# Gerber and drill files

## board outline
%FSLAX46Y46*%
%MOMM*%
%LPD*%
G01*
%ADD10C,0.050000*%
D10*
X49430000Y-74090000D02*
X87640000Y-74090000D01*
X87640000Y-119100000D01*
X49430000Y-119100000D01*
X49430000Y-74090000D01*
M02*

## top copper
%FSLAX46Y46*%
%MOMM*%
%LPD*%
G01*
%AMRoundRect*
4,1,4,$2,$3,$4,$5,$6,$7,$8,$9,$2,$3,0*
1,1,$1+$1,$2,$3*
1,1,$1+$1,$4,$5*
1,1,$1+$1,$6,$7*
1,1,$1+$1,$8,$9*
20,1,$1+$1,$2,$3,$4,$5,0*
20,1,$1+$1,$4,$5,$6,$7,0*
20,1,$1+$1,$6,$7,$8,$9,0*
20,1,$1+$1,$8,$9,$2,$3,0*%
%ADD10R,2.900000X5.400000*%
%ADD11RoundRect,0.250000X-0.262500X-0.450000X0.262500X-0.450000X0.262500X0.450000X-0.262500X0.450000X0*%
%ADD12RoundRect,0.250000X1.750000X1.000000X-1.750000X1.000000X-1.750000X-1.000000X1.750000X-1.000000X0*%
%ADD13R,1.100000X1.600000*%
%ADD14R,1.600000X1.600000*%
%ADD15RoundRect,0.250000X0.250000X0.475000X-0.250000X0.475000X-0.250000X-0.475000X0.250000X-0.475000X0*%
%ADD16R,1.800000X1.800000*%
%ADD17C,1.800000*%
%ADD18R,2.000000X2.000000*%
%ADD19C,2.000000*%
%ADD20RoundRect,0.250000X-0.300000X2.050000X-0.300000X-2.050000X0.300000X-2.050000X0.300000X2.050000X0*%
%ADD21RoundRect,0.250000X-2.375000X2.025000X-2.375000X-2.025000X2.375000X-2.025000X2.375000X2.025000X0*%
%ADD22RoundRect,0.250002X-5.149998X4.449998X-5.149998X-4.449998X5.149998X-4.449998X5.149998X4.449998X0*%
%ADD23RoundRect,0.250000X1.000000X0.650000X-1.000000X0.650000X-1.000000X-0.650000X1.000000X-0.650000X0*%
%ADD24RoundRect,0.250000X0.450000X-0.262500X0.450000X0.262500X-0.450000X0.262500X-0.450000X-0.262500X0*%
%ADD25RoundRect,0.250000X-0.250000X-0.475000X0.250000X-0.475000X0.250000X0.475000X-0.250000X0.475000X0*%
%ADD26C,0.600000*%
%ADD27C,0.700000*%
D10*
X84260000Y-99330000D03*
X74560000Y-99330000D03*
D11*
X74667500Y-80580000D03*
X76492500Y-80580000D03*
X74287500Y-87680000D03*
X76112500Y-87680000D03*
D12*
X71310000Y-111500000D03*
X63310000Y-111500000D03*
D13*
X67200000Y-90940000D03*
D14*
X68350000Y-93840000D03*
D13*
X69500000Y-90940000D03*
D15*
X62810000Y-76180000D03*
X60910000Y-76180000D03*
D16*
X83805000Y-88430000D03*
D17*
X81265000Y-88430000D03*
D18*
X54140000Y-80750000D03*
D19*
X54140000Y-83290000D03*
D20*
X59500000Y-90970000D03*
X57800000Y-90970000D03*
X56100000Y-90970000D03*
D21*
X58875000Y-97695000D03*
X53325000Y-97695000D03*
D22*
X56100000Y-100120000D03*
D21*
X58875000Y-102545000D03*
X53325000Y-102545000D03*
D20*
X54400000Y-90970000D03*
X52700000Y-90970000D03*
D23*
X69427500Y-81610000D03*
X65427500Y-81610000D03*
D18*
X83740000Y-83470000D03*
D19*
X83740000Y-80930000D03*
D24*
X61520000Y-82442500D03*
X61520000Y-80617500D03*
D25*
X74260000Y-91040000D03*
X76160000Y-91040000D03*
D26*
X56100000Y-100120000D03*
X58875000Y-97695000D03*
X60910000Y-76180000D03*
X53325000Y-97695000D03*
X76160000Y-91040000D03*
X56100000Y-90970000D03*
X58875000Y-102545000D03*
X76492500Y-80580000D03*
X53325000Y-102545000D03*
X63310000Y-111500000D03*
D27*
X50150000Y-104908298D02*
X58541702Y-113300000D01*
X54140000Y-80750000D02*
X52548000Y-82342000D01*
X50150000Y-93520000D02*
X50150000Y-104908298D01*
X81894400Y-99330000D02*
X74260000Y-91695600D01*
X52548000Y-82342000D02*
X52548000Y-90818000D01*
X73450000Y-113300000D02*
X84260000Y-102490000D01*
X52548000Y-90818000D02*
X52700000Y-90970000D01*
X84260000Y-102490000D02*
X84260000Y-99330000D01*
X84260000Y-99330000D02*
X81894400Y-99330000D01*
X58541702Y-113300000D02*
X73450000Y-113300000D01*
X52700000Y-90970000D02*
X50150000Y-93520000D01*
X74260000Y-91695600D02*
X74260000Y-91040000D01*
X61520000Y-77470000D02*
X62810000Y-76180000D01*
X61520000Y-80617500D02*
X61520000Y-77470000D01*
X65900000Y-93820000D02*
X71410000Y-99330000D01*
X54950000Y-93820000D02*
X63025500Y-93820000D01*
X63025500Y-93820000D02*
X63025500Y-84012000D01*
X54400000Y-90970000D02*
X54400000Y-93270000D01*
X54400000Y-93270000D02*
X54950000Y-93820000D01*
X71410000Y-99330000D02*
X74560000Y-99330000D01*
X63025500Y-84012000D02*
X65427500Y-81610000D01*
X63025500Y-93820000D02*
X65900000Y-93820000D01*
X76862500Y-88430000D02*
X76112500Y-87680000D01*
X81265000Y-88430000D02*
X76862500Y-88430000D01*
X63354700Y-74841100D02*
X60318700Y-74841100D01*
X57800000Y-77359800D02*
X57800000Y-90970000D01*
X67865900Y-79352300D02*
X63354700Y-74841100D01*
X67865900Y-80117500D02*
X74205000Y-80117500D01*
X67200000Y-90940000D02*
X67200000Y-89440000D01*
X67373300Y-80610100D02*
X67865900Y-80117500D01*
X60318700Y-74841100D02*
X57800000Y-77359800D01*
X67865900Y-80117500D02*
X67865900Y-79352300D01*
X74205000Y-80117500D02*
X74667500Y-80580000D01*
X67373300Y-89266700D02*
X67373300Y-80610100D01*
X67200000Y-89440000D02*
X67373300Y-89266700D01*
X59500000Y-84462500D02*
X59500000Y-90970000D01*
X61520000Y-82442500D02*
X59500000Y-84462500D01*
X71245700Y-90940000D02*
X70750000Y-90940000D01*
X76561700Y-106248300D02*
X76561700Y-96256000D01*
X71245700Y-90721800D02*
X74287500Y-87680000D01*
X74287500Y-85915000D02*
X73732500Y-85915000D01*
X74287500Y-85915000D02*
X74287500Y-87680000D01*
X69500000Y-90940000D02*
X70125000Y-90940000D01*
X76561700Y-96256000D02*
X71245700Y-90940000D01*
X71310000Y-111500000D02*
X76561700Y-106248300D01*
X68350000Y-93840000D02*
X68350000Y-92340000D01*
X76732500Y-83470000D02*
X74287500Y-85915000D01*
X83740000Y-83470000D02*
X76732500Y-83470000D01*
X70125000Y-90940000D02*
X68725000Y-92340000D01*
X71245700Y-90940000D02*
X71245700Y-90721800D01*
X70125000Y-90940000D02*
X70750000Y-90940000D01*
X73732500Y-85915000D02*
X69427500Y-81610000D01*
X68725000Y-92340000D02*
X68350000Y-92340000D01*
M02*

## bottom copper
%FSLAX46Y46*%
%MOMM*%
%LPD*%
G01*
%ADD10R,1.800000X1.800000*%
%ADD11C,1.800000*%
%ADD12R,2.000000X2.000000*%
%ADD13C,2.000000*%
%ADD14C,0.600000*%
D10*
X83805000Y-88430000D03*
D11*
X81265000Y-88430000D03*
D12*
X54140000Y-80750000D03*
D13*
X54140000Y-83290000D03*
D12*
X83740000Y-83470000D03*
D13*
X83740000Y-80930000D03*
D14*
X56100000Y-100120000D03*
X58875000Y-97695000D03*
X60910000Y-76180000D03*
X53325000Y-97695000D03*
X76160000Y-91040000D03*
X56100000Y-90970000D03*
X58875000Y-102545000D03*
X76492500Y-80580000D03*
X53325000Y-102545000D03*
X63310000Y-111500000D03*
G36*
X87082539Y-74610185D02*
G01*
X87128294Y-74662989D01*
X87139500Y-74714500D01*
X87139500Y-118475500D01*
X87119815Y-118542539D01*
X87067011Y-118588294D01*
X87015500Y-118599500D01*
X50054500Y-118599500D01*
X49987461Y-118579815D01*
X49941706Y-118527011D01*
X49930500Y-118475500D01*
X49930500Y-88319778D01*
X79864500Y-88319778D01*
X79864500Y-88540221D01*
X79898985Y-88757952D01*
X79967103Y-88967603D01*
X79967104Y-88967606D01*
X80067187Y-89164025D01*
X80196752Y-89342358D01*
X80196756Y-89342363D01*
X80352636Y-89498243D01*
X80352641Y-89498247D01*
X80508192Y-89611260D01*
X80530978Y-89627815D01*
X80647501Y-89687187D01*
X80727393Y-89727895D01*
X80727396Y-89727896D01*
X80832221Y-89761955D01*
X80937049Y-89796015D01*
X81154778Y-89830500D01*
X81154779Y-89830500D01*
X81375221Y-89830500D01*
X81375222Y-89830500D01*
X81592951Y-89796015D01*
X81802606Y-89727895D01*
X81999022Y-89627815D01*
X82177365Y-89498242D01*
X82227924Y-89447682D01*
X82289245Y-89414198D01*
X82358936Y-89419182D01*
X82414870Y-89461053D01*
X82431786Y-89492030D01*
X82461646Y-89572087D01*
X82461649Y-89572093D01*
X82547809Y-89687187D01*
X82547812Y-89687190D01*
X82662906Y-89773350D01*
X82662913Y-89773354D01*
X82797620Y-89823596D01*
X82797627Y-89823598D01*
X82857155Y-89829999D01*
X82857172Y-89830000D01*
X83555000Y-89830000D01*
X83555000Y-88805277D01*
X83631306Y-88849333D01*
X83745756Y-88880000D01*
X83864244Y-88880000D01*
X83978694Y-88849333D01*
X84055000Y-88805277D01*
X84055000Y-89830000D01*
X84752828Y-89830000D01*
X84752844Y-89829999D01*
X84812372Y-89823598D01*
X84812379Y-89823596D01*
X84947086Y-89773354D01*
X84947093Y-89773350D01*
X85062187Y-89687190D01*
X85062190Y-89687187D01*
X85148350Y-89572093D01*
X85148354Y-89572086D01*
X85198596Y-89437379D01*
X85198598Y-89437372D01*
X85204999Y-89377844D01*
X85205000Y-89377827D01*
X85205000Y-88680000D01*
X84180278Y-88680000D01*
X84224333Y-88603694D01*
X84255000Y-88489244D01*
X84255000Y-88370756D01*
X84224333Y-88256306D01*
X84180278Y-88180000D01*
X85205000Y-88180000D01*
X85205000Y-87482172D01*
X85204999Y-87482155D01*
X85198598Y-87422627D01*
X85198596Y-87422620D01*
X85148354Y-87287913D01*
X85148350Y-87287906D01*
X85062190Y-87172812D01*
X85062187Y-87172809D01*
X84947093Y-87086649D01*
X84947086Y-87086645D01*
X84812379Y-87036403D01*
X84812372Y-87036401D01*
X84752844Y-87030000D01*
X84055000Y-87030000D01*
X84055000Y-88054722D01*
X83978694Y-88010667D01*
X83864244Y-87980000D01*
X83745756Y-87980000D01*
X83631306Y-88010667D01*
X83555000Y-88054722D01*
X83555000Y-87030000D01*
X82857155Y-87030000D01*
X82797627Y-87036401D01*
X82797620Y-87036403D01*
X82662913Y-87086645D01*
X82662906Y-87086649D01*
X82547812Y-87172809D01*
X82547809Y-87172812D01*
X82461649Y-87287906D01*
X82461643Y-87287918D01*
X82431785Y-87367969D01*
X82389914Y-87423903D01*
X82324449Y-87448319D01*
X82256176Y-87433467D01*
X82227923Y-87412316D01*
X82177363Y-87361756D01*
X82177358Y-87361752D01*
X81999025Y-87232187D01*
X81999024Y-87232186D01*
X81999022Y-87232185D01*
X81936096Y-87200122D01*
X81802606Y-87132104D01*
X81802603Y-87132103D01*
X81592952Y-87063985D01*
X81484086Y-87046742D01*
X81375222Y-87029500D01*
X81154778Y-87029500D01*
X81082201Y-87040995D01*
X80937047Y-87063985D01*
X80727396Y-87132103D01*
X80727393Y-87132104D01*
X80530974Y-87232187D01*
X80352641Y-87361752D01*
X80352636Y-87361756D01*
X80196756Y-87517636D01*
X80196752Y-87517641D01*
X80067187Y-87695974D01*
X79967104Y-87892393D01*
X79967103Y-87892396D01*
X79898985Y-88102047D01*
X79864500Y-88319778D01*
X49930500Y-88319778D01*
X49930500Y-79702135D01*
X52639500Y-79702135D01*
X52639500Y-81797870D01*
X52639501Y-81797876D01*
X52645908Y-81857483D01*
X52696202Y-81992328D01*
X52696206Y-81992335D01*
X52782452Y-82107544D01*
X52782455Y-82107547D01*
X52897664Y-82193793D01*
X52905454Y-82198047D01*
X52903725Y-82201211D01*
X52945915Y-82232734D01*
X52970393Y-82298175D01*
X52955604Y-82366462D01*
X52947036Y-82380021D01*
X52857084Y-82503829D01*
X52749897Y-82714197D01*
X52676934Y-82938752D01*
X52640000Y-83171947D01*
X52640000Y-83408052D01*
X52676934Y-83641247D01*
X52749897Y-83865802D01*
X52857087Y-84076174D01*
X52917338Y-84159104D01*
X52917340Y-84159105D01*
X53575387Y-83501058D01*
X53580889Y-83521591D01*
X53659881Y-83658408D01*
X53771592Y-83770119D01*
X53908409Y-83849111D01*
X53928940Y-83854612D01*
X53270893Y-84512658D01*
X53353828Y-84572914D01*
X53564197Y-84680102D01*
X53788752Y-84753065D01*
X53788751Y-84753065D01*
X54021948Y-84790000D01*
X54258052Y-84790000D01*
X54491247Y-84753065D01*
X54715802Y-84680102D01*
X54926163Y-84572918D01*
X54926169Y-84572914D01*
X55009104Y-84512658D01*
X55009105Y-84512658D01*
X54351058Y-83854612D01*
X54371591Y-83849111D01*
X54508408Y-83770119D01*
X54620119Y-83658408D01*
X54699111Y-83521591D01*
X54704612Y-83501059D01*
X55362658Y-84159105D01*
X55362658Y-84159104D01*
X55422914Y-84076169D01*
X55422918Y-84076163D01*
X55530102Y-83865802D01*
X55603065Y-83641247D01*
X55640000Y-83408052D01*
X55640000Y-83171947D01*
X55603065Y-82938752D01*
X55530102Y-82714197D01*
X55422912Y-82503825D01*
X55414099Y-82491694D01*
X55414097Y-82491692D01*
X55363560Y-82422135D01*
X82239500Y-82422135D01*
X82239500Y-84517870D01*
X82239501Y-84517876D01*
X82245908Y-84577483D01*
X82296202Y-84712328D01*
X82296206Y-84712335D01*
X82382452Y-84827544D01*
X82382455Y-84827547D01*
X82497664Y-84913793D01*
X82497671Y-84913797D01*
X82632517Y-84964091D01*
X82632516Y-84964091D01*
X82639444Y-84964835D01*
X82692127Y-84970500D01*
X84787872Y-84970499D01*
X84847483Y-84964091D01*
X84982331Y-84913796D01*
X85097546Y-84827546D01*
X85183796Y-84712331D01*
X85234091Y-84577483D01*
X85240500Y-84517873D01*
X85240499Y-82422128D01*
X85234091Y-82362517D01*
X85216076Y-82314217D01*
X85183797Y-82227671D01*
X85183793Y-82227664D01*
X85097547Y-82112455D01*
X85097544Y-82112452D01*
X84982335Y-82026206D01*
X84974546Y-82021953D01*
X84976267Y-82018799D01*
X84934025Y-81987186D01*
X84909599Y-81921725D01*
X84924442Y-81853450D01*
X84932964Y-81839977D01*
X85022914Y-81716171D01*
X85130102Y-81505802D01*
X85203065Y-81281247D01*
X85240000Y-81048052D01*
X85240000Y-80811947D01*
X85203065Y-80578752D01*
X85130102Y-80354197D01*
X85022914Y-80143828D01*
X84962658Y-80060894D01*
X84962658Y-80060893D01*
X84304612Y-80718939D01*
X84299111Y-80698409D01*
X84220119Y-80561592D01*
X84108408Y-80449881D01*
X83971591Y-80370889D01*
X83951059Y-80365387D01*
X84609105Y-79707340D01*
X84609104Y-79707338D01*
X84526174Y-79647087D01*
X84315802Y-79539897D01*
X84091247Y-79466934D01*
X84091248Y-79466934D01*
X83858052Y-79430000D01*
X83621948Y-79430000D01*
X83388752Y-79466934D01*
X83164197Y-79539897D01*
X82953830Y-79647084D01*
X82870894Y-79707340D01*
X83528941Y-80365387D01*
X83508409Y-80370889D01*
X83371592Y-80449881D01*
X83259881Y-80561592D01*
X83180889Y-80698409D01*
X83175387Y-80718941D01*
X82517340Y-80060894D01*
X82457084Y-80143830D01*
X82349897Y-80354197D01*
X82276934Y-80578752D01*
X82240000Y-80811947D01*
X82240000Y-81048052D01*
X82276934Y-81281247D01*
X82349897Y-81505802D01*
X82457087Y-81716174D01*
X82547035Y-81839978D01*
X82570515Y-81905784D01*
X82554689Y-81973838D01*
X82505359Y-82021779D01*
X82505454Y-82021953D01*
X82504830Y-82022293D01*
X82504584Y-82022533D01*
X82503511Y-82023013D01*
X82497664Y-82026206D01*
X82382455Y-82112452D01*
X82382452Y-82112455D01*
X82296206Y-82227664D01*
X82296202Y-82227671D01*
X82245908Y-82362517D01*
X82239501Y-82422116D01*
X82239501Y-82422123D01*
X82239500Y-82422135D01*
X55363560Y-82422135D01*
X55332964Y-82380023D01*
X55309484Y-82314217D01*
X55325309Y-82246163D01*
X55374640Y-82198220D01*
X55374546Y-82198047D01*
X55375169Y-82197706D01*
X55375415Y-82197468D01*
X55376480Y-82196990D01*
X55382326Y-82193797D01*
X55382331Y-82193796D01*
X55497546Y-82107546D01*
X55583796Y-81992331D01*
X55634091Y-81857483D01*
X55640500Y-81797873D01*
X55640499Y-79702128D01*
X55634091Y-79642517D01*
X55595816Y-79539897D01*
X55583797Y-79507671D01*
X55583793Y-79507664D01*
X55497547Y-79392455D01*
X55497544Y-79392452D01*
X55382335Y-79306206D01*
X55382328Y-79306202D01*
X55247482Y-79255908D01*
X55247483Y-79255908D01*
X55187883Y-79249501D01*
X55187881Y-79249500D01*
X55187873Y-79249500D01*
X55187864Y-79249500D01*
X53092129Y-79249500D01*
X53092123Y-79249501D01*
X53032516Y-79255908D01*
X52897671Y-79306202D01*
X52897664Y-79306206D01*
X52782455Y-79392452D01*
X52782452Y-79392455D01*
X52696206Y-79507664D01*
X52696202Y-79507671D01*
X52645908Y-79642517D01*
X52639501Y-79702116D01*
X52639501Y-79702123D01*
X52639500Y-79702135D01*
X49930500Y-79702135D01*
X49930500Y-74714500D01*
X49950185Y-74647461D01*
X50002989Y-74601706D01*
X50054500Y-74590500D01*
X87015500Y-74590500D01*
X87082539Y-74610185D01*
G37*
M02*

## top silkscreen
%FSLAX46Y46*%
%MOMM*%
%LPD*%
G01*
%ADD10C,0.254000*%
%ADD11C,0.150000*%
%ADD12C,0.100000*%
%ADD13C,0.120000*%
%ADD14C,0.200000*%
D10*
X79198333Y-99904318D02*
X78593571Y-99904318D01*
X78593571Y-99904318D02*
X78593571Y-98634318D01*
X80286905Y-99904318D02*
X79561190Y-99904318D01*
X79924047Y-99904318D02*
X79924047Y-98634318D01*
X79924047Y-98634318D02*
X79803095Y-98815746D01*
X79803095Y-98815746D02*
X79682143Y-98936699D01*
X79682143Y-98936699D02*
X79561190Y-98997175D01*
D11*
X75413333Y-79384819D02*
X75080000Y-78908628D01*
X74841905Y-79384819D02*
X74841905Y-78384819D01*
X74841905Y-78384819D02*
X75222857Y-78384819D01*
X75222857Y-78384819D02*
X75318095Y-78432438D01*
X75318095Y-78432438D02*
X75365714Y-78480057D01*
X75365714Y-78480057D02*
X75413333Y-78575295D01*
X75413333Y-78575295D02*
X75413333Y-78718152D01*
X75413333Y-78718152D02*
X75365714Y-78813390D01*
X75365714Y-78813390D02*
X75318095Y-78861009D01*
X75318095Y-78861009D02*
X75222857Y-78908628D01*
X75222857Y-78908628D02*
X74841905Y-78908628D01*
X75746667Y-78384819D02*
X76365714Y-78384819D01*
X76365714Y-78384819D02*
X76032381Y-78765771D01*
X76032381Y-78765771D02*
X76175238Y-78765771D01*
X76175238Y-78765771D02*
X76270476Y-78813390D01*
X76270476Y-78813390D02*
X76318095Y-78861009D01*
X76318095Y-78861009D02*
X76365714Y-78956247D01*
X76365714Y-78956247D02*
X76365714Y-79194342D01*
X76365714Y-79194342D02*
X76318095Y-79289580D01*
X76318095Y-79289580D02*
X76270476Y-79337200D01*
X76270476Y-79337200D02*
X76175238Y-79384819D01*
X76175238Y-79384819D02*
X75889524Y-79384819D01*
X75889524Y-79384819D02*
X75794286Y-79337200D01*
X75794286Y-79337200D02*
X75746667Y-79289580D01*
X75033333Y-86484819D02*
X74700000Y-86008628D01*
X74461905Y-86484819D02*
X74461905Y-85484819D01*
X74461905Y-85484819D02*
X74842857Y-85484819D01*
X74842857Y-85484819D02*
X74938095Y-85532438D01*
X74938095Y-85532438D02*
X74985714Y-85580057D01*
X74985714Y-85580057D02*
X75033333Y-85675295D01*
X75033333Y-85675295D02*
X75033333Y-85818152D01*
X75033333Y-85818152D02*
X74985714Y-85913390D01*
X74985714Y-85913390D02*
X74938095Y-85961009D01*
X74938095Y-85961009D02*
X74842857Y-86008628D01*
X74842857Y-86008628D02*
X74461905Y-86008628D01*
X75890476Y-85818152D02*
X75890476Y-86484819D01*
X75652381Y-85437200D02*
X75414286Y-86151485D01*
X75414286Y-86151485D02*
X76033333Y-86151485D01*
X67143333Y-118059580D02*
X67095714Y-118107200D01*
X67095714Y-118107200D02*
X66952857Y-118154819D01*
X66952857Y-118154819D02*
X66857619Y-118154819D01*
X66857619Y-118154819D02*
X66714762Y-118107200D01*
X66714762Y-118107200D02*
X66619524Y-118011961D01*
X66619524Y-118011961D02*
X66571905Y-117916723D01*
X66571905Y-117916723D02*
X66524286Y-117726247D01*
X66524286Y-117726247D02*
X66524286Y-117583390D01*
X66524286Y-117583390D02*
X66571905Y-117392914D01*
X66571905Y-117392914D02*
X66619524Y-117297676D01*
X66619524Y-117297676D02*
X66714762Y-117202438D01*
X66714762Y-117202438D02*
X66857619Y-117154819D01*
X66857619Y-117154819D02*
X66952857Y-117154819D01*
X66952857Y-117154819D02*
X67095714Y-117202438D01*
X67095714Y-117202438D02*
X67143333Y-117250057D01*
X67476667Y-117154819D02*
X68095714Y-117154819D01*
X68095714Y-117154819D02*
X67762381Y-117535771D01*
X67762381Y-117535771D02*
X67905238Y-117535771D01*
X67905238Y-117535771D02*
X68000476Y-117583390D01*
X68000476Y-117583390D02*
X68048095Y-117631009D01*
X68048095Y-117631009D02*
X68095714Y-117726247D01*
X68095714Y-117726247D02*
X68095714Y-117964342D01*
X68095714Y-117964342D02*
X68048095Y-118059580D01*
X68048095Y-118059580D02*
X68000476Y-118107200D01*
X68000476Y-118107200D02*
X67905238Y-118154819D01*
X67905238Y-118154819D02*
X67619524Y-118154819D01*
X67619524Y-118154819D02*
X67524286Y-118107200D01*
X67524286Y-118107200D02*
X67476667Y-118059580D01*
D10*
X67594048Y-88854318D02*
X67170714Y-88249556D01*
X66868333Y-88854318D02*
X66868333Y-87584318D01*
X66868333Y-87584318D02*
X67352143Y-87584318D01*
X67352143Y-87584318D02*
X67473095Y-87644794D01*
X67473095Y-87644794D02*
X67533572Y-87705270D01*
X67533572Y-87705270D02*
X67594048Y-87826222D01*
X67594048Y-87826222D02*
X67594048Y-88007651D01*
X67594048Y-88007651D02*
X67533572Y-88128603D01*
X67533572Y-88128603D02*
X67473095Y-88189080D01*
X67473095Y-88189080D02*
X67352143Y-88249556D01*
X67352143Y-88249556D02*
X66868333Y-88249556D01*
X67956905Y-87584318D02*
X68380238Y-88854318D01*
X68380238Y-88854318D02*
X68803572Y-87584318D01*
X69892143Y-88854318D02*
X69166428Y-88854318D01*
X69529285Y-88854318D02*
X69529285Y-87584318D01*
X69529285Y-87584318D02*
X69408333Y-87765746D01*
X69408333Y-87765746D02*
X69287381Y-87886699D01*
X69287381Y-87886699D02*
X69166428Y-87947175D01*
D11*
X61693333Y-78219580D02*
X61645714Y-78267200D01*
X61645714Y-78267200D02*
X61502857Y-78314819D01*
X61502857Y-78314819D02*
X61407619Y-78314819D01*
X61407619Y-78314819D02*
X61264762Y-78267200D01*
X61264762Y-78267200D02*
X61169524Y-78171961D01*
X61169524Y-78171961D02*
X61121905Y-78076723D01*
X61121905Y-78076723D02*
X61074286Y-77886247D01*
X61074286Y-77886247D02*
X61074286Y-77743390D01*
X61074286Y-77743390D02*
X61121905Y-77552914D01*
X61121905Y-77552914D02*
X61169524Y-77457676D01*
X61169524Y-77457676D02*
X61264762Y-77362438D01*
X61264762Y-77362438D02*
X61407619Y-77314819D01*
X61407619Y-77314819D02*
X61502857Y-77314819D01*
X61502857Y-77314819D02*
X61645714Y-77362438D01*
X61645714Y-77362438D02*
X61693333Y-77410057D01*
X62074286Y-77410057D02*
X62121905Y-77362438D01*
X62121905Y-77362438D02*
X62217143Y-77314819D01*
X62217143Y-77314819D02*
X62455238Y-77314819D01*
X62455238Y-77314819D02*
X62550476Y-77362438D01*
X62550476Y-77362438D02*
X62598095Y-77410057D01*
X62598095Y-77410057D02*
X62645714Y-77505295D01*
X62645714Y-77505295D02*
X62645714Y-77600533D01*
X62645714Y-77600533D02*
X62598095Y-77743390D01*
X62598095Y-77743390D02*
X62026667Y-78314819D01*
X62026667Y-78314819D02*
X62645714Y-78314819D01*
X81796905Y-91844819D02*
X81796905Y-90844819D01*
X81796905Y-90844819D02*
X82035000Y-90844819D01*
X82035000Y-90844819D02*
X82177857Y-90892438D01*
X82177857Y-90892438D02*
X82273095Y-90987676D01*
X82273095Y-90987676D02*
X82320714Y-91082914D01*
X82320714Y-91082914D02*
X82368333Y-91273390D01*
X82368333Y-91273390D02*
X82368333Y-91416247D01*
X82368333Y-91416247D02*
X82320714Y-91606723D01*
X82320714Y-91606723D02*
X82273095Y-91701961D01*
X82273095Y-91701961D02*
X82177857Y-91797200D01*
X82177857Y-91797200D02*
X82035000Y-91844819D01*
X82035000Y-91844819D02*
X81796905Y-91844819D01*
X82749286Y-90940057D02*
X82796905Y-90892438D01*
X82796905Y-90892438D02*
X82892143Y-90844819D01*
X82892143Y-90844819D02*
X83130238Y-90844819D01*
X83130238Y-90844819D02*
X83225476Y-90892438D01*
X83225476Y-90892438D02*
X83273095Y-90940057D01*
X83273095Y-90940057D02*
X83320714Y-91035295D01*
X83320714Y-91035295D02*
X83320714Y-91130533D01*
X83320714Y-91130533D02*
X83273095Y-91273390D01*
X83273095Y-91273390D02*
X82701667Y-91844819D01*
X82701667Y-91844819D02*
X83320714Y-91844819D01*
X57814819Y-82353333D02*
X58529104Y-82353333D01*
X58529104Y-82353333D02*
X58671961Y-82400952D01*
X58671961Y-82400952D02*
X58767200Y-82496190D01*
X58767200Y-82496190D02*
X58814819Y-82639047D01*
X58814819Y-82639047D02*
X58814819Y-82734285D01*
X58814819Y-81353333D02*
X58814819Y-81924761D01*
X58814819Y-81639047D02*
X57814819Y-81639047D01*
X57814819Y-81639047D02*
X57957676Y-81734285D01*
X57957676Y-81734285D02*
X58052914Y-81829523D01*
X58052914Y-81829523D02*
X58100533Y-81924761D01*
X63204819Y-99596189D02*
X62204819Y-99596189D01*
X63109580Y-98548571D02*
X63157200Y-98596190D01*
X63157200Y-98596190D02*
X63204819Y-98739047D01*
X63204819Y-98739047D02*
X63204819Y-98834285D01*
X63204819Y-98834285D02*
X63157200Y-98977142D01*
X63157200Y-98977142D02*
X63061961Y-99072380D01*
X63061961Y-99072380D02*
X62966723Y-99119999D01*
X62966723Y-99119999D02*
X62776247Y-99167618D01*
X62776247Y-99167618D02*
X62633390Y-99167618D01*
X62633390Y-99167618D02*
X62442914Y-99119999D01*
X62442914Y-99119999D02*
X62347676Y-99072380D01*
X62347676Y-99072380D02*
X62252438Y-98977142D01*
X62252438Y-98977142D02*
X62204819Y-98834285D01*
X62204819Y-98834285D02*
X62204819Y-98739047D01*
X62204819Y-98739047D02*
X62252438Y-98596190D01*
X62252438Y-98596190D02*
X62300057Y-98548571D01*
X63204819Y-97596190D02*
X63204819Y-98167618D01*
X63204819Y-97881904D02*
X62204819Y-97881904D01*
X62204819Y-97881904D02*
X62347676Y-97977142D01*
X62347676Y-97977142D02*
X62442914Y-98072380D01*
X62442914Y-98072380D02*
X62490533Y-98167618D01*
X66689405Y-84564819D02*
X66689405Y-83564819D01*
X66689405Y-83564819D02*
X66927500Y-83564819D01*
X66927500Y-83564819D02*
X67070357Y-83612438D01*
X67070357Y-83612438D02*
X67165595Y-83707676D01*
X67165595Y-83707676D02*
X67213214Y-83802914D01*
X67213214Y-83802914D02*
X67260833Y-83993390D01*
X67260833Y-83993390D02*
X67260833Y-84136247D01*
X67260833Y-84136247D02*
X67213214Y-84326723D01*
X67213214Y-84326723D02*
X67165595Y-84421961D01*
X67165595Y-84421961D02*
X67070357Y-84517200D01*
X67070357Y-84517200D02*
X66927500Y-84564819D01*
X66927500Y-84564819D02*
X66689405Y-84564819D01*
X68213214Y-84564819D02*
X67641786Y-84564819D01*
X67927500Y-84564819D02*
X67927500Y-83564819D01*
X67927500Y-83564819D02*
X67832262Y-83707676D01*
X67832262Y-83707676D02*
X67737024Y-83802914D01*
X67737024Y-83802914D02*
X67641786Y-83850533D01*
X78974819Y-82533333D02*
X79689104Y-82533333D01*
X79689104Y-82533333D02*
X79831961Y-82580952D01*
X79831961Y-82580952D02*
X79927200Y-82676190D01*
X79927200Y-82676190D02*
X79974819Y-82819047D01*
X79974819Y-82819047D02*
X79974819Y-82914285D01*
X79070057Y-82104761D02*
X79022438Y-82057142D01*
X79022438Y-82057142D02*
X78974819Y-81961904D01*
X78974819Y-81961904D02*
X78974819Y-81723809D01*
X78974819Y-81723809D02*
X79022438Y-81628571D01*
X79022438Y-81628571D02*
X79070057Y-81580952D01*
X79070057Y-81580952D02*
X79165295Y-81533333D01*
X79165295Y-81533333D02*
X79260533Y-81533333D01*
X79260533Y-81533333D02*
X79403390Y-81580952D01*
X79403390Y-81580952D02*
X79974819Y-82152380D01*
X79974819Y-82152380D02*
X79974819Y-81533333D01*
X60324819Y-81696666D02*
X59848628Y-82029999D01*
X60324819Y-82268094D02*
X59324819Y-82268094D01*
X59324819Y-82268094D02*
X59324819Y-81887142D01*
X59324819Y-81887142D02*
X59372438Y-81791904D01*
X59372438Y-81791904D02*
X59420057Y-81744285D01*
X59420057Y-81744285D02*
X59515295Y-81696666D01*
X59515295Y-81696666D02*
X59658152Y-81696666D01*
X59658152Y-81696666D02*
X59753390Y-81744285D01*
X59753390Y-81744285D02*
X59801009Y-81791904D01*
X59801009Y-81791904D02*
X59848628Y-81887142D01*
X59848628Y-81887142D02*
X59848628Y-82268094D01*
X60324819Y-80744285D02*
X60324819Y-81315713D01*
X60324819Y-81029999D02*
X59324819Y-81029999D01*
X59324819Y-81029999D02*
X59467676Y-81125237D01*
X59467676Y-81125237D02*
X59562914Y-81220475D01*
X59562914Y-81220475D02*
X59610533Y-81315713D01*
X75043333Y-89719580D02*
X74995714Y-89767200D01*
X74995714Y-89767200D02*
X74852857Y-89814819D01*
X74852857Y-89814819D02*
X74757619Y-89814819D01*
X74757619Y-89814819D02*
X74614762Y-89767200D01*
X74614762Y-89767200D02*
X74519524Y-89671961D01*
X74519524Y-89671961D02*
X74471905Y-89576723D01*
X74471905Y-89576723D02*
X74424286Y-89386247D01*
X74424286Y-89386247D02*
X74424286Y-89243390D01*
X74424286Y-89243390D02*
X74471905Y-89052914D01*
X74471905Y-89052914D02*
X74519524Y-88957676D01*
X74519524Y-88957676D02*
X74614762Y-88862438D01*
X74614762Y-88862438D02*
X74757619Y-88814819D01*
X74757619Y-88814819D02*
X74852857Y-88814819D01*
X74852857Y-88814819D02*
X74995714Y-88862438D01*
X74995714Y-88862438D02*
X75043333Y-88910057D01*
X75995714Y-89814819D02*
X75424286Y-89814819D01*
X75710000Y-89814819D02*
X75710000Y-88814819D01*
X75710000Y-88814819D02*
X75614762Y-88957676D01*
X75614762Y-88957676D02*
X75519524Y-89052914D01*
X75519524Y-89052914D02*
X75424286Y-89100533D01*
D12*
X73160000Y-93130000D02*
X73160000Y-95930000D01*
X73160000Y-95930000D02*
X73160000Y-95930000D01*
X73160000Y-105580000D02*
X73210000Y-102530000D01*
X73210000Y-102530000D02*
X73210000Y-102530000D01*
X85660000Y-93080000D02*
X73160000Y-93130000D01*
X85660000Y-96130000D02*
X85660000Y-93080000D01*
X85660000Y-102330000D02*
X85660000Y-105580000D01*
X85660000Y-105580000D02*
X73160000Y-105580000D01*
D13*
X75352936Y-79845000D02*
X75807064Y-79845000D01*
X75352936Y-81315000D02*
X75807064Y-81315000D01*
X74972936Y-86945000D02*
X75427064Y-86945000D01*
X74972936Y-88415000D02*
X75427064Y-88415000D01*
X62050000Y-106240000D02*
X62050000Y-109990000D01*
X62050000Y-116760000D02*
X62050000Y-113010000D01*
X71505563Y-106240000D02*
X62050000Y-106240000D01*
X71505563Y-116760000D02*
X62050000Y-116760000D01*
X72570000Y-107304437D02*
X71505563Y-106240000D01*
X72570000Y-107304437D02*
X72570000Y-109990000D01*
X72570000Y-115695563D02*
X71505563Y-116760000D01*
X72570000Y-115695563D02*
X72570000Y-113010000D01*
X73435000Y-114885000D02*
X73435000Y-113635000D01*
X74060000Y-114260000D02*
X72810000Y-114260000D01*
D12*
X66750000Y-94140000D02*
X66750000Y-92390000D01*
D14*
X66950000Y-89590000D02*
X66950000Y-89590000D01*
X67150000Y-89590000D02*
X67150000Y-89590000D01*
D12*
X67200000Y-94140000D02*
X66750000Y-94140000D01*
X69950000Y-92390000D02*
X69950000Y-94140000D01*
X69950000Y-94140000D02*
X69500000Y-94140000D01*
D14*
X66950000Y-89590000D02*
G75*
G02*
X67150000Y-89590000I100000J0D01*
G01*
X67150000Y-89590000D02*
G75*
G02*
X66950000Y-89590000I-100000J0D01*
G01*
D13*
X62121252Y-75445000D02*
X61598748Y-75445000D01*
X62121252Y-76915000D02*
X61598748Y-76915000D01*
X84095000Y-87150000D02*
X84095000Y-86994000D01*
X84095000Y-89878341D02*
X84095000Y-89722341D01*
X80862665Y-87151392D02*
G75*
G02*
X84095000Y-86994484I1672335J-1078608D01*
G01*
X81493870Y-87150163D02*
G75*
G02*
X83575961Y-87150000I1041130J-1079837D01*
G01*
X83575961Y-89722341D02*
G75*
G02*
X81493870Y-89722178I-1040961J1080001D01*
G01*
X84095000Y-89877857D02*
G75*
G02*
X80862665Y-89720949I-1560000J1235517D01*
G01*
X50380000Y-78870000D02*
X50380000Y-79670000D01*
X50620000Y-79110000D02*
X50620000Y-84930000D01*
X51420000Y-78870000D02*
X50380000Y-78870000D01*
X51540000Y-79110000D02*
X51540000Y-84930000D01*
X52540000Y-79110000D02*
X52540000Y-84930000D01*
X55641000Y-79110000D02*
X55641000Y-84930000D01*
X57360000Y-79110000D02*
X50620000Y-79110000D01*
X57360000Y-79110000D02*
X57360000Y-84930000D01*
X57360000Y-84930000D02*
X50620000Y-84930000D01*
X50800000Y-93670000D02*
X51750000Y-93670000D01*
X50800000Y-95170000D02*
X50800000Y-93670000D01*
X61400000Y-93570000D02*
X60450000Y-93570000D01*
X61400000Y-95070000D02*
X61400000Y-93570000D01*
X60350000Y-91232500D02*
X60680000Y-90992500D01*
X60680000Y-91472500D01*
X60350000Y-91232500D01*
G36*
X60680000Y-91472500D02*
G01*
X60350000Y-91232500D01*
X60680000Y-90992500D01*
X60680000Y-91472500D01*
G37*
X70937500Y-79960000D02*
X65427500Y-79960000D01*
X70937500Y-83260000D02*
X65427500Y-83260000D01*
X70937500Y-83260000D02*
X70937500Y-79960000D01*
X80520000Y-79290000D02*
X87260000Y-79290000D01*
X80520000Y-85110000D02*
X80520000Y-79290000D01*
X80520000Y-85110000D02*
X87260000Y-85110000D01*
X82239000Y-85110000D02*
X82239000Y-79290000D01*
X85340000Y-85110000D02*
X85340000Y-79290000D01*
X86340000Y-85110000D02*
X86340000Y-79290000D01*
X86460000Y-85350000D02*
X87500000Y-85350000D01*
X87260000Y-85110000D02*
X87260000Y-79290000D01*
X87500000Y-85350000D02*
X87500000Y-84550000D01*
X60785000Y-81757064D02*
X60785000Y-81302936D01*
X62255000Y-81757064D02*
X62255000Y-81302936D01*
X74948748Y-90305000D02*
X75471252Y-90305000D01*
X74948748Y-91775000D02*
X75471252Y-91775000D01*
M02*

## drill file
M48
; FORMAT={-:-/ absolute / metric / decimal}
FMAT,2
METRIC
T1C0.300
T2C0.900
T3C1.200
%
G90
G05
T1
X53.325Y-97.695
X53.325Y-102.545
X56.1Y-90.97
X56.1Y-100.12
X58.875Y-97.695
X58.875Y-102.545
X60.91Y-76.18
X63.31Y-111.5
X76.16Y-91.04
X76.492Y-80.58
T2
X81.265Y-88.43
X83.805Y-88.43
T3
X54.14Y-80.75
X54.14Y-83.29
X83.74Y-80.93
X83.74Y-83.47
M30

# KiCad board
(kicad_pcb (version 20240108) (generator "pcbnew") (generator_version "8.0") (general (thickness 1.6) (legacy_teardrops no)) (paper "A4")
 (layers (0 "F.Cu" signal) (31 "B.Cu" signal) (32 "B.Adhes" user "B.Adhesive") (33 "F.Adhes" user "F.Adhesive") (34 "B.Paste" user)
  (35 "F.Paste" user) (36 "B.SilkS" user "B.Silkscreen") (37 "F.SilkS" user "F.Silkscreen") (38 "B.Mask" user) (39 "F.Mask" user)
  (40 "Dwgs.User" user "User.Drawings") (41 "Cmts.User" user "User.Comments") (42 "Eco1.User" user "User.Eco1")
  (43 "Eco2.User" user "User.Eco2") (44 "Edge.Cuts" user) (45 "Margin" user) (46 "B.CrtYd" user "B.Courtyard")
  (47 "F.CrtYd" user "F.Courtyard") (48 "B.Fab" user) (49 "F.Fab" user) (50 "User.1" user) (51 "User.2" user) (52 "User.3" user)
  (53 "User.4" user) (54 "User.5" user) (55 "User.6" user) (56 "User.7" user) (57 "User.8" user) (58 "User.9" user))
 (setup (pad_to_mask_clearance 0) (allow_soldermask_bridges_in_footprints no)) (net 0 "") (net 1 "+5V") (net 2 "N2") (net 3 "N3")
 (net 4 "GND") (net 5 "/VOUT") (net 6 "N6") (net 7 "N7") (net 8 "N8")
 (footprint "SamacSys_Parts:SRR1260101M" (layer "F.Cu") (at 79.41 99.33 180)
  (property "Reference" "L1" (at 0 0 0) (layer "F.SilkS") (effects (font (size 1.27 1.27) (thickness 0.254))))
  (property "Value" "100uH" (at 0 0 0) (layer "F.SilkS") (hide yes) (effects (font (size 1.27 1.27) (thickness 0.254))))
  (fp_line (start 6.25 6.2) (end 6.25 3.4) (stroke (width 0.1) (type solid)) (layer "F.SilkS"))
  (fp_line (start 6.25 3.4) (end 6.25 3.4) (stroke (width 0.1) (type solid)) (layer "F.SilkS"))
  (fp_line (start 6.25 -6.25) (end 6.2 -3.2) (stroke (width 0.1) (type solid)) (layer "F.SilkS"))
  (fp_line (start 6.2 -3.2) (end 6.2 -3.2) (stroke (width 0.1) (type solid)) (layer "F.SilkS"))
  (fp_line (start -6.25 6.25) (end 6.25 6.2) (stroke (width 0.1) (type solid)) (layer "F.SilkS"))
  (fp_line (start -6.25 3.2) (end -6.25 6.25) (stroke (width 0.1) (type solid)) (layer "F.SilkS"))
  (fp_line (start -6.25 -3) (end -6.25 -6.25) (stroke (width 0.1) (type solid)) (layer "F.SilkS"))
  (fp_line (start -6.25 -6.25) (end 6.25 -6.25) (stroke (width 0.1) (type solid)) (layer "F.SilkS"))
  (pad "1" smd rect (at -4.85 0 180) (size 2.9 5.4) (layers "F.Cu" "F.Paste" "F.Mask") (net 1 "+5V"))
  (pad "2" smd rect (at 4.85 0 180) (size 2.9 5.4) (layers "F.Cu" "F.Paste" "F.Mask") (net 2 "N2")))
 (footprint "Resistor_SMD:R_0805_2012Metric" (layer "F.Cu") (at 75.58 80.58)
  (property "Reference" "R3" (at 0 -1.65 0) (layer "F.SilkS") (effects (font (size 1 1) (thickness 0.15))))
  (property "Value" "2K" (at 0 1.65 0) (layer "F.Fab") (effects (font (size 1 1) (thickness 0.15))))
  (fp_line (start -0.227064 -0.735) (end 0.227064 -0.735) (stroke (width 0.12) (type solid)) (layer "F.SilkS"))
  (fp_line (start -0.227064 0.735) (end 0.227064 0.735) (stroke (width 0.12) (type solid)) (layer "F.SilkS"))
  (pad "1" smd roundrect (at -0.9125 0) (size 1.025 1.4) (layers "F.Cu" "F.Paste" "F.Mask") (roundrect_rratio 0.243902) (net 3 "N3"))
  (pad "2" smd roundrect (at 0.9125 0) (size 1.025 1.4) (layers "F.Cu" "F.Paste" "F.Mask") (roundrect_rratio 0.243902) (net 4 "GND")))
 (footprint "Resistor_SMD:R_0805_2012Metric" (layer "F.Cu") (at 75.2 87.68)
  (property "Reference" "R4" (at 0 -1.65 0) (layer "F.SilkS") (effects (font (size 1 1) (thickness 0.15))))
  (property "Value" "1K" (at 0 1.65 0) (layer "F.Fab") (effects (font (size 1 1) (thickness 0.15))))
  (fp_line (start -0.227064 -0.735) (end 0.227064 -0.735) (stroke (width 0.12) (type solid)) (layer "F.SilkS"))
  (fp_line (start -0.227064 0.735) (end 0.227064 0.735) (stroke (width 0.12) (type solid)) (layer "F.SilkS"))
  (pad "1" smd roundrect (at -0.9125 0) (size 1.025 1.4) (layers "F.Cu" "F.Paste" "F.Mask") (roundrect_rratio 0.243902) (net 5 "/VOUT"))
  (pad "2" smd roundrect (at 0.9125 0) (size 1.025 1.4) (layers "F.Cu" "F.Paste" "F.Mask") (roundrect_rratio 0.243902) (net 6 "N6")))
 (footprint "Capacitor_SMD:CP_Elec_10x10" (layer "F.Cu") (at 67.31 111.5 180)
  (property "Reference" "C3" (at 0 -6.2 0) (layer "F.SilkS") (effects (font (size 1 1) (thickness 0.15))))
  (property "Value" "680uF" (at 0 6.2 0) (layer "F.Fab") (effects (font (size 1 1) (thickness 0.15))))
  (fp_line (start 5.26 5.26) (end 5.26 1.51) (stroke (width 0.12) (type solid)) (layer "F.SilkS"))
  (fp_line (start 5.26 -5.26) (end 5.26 -1.51) (stroke (width 0.12) (type solid)) (layer "F.SilkS"))
  (fp_line (start -4.195563 5.26) (end 5.26 5.26) (stroke (width 0.12) (type solid)) (layer "F.SilkS"))
  (fp_line (start -4.195563 -5.26) (end 5.26 -5.26) (stroke (width 0.12) (type solid)) (layer "F.SilkS"))
  (fp_line (start -5.26 4.195563) (end -4.195563 5.26) (stroke (width 0.12) (type solid)) (layer "F.SilkS"))
  (fp_line (start -5.26 4.195563) (end -5.26 1.51) (stroke (width 0.12) (type solid)) (layer "F.SilkS"))
  (fp_line (start -5.26 -4.195563) (end -4.195563 -5.26) (stroke (width 0.12) (type solid)) (layer "F.SilkS"))
  (fp_line (start -5.26 -4.195563) (end -5.26 -1.51) (stroke (width 0.12) (type solid)) (layer "F.SilkS"))
  (fp_line (start -6.125 -3.385) (end -6.125 -2.135) (stroke (width 0.12) (type solid)) (layer "F.SilkS"))
  (fp_line (start -6.75 -2.76) (end -5.5 -2.76) (stroke (width 0.12) (type solid)) (layer "F.SilkS"))
  (pad "1" smd roundrect (at -4 0 180) (size 4 2.5) (layers "F.Cu" "F.Paste" "F.Mask") (roundrect_rratio 0.1) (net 5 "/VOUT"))
  (pad "2" smd roundrect (at 4 0 180) (size 4 2.5) (layers "F.Cu" "F.Paste" "F.Mask") (roundrect_rratio 0.1) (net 4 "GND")))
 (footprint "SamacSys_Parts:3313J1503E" (layer "F.Cu") (at 68.35 92.39 180)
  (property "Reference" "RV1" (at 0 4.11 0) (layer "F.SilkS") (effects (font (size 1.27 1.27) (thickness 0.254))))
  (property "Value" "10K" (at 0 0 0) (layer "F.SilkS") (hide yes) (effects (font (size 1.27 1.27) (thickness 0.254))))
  (fp_line (start 1.6 -1.75) (end 1.6 0) (stroke (width 0.1) (type solid)) (layer "F.SilkS"))
  (fp_line (start 1.4 2.8) (end 1.4 2.8) (stroke (width 0.2) (type solid)) (layer "F.SilkS"))
  (fp_line (start 1.2 2.8) (end 1.2 2.8) (stroke (width 0.2) (type solid)) (layer "F.SilkS"))
  (fp_line (start 1.15 -1.75) (end 1.6 -1.75) (stroke (width 0.1) (type solid)) (layer "F.SilkS"))
  (fp_line (start -1.6 0) (end -1.6 -1.75) (stroke (width 0.1) (type solid)) (layer "F.SilkS"))
  (fp_line (start -1.6 -1.75) (end -1.15 -1.75) (stroke (width 0.1) (type solid)) (layer "F.SilkS"))
  (fp_arc (start 1.4 2.8) (mid 1.3 2.9) (end 1.2 2.8) (stroke (width 0.2) (type solid)) (layer "F.SilkS"))
  (fp_arc (start 1.2 2.8) (mid 1.3 2.7) (end 1.4 2.8) (stroke (width 0.2) (type solid)) (layer "F.SilkS"))
  (pad "1" smd rect (at 1.15 1.45 180) (size 1.1 1.6) (layers "F.Cu" "F.Paste" "F.Mask") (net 3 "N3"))
  (pad "2" smd rect (at 0 -1.45 270) (size 1.6 1.6) (layers "F.Cu" "F.Paste" "F.Mask") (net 5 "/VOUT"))
  (pad "3" smd rect (at -1.15 1.45 180) (size 1.1 1.6) (layers "F.Cu" "F.Paste" "F.Mask") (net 5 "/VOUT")))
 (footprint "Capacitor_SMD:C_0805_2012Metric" (layer "F.Cu") (at 61.86 76.18 180)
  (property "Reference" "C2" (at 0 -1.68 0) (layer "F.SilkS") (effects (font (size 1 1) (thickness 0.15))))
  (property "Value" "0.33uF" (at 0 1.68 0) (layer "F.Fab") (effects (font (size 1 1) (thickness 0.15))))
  (fp_line (start -0.261252 0.735) (end 0.261252 0.735) (stroke (width 0.12) (type solid)) (layer "F.SilkS"))
  (fp_line (start -0.261252 -0.735) (end 0.261252 -0.735) (stroke (width 0.12) (type solid)) (layer "F.SilkS"))
  (pad "1" smd roundrect (at -0.95 0 180) (size 1 1.45) (layers "F.Cu" "F.Paste" "F.Mask") (roundrect_rratio 0.25) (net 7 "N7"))
  (pad "2" smd roundrect (at 0.95 0 180) (size 1 1.45) (layers "F.Cu" "F.Paste" "F.Mask") (roundrect_rratio 0.25) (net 4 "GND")))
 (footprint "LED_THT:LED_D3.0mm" (layer "F.Cu") (at 83.805 88.43 180)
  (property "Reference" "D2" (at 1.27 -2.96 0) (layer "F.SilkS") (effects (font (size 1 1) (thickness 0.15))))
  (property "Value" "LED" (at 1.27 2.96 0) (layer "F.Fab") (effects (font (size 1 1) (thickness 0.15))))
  (fp_line (start -0.29 1.28) (end -0.29 1.436) (stroke (width 0.12) (type solid)) (layer "F.SilkS"))
  (fp_line (start -0.29 -1.448341) (end -0.29 -1.292341) (stroke (width 0.12) (type solid)) (layer "F.SilkS"))
  (fp_arc (start 2.942335 1.278608) (mid 1.366487 2.187659) (end -0.29 1.435516) (stroke (width 0.12) (type solid)) (layer "F.SilkS"))
  (fp_arc (start 2.31113 1.279837) (mid 1.270117 1.7) (end 0.229039 1.28) (stroke (width 0.12) (type solid)) (layer "F.SilkS"))
  (fp_arc (start 0.229039 -1.292341) (mid 1.270117 -1.712341) (end 2.31113 -1.292178) (stroke (width 0.12) (type solid)) (layer "F.SilkS"))
  (fp_arc (start -0.29 -1.447857) (mid 1.366487 -2.2) (end 2.942335 -1.290949) (stroke (width 0.12) (type solid)) (layer "F.SilkS"))
  (pad "1" thru_hole rect (at 0 0 180) (size 1.8 1.8) (drill 0.9) (layers "*.Cu" "*.Mask") (remove_unused_layers no) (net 4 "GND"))
  (pad "2" thru_hole circle (at 2.54 0 180) (size 1.8 1.8) (drill 0.9) (layers "*.Cu" "*.Mask") (remove_unused_layers no) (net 6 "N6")))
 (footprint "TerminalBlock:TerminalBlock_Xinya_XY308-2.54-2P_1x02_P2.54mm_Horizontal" (layer "F.Cu") (at 54.14 80.75 -90)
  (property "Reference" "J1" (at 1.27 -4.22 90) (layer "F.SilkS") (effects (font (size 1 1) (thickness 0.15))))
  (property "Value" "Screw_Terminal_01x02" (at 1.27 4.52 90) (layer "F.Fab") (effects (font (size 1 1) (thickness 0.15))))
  (fp_line (start -1.88 3.76) (end -1.08 3.76) (stroke (width 0.12) (type solid)) (layer "F.SilkS"))
  (fp_line (start -1.64 3.52) (end 4.18 3.52) (stroke (width 0.12) (type solid)) (layer "F.SilkS"))
  (fp_line (start -1.88 2.72) (end -1.88 3.76) (stroke (width 0.12) (type solid)) (layer "F.SilkS"))
  (fp_line (start -1.64 2.6) (end 4.18 2.6) (stroke (width 0.12) (type solid)) (layer "F.SilkS"))
  (fp_line (start -1.64 1.6) (end 4.18 1.6) (stroke (width 0.12) (type solid)) (layer "F.SilkS"))
  (fp_line (start -1.64 -1.501) (end 4.18 -1.501) (stroke (width 0.12) (type solid)) (layer "F.SilkS"))
  (fp_line (start -1.64 -3.22) (end -1.64 3.52) (stroke (width 0.12) (type solid)) (layer "F.SilkS"))
  (fp_line (start -1.64 -3.22) (end 4.18 -3.22) (stroke (width 0.12) (type solid)) (layer "F.SilkS"))
  (fp_line (start 4.18 -3.22) (end 4.18 3.52) (stroke (width 0.12) (type solid)) (layer "F.SilkS"))
  (pad "1" thru_hole rect (at 0 0 270) (size 2 2) (drill 1.2) (layers "*.Cu" "*.Mask") (remove_unused_layers no) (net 1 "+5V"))
  (pad "2" thru_hole circle (at 2.54 0 270) (size 2 2) (drill 1.2) (layers "*.Cu" "*.Mask") (remove_unused_layers no) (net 4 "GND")))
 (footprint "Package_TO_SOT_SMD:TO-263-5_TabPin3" (layer "F.Cu") (at 56.1 98.62 -90)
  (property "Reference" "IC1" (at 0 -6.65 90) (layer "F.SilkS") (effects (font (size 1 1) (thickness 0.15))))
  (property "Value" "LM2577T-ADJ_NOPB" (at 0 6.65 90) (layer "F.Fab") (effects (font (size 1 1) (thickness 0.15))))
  (fp_line (start -4.95 5.3) (end -4.95 4.35) (stroke (width 0.12) (type solid)) (layer "F.SilkS"))
  (fp_line (start -3.45 5.3) (end -4.95 5.3) (stroke (width 0.12) (type solid)) (layer "F.SilkS"))
  (fp_line (start -5.05 -5.3) (end -5.05 -4.35) (stroke (width 0.12) (type solid)) (layer "F.SilkS"))
  (fp_line (start -3.55 -5.3) (end -5.05 -5.3) (stroke (width 0.12) (type solid)) (layer "F.SilkS"))
  (fp_poly
   (pts (xy -7.3875 -4.25) (xy -7.6275 -4.58) (xy -7.1475 -4.58) (xy -7.3875 -4.25)) (stroke (width 0.12) (type solid)) (fill solid)
   (layer "F.SilkS"))
  (pad "1" smd roundrect (at -7.65 -3.4 270) (size 4.6 1.1) (layers "F.Cu" "F.Paste" "F.Mask") (roundrect_rratio 0.227273) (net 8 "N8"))
  (pad "2" smd roundrect (at -7.65 -1.7 270) (size 4.6 1.1) (layers "F.Cu" "F.Paste" "F.Mask") (roundrect_rratio 0.227273) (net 3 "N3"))
  (pad "3" smd roundrect (at -7.65 0 270) (size 4.6 1.1) (layers "F.Cu" "F.Paste" "F.Mask") (roundrect_rratio 0.227273) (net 4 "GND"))
  (pad "3" smd roundrect (at -0.925 -2.775 270) (size 4.55 5.25) (layers "F.Cu" "F.Paste") (roundrect_rratio 0.054945) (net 4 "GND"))
  (pad "3" smd roundrect (at -0.925 2.775 270) (size 4.55 5.25) (layers "F.Cu" "F.Paste") (roundrect_rratio 0.054945) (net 4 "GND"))
  (pad "3" smd roundrect (at 1.5 0 270) (size 9.4 10.8) (layers "F.Cu" "F.Mask") (roundrect_rratio 0.026596) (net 4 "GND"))
  (pad "3" smd roundrect (at 3.925 -2.775 270) (size 4.55 5.25) (layers "F.Cu" "F.Paste") (roundrect_rratio 0.054945) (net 4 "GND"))
  (pad "3" smd roundrect (at 3.925 2.775 270) (size 4.55 5.25) (layers "F.Cu" "F.Paste") (roundrect_rratio 0.054945) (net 4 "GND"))
  (pad "4" smd roundrect (at -7.65 1.7 270) (size 4.6 1.1) (layers "F.Cu" "F.Paste" "F.Mask") (roundrect_rratio 0.227273) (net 2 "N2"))
  (pad "5" smd roundrect (at -7.65 3.4 270) (size 4.6 1.1) (layers "F.Cu" "F.Paste" "F.Mask") (roundrect_rratio 0.227273) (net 1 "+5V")))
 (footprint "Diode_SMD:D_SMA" (layer "F.Cu") (at 67.4275 81.61 180)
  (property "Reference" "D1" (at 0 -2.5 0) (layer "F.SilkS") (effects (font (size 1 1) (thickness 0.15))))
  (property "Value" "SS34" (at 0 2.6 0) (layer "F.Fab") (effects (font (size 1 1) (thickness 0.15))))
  (fp_line (start -3.51 1.65) (end 2 1.65) (stroke (width 0.12) (type solid)) (layer "F.SilkS"))
  (fp_line (start -3.51 -1.65) (end 2 -1.65) (stroke (width 0.12) (type solid)) (layer "F.SilkS"))
  (fp_line (start -3.51 -1.65) (end -3.51 1.65) (stroke (width 0.12) (type solid)) (layer "F.SilkS"))
  (pad "1" smd roundrect (at -2 0 180) (size 2.5 1.8) (layers "F.Cu" "F.Paste" "F.Mask") (roundrect_rratio 0.1388888889) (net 5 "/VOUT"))
  (pad "2" smd roundrect (at 2 0 180) (size 2.5 1.8) (layers "F.Cu" "F.Paste" "F.Mask") (roundrect_rratio 0.1388888889) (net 2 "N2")))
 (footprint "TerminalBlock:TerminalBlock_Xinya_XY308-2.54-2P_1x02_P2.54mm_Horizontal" (layer "F.Cu") (at 83.74 83.47 90)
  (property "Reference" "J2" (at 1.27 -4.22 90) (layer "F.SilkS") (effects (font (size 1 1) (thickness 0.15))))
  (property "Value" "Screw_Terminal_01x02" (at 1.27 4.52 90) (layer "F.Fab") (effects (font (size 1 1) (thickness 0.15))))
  (fp_line (start 4.18 -3.22) (end 4.18 3.52) (stroke (width 0.12) (type solid)) (layer "F.SilkS"))
  (fp_line (start -1.64 -3.22) (end 4.18 -3.22) (stroke (width 0.12) (type solid)) (layer "F.SilkS"))
  (fp_line (start -1.64 -3.22) (end -1.64 3.52) (stroke (width 0.12) (type solid)) (layer "F.SilkS"))
  (fp_line (start -1.64 -1.501) (end 4.18 -1.501) (stroke (width 0.12) (type solid)) (layer "F.SilkS"))
  (fp_line (start -1.64 1.6) (end 4.18 1.6) (stroke (width 0.12) (type solid)) (layer "F.SilkS"))
  (fp_line (start -1.64 2.6) (end 4.18 2.6) (stroke (width 0.12) (type solid)) (layer "F.SilkS"))
  (fp_line (start -1.88 2.72) (end -1.88 3.76) (stroke (width 0.12) (type solid)) (layer "F.SilkS"))
  (fp_line (start -1.64 3.52) (end 4.18 3.52) (stroke (width 0.12) (type solid)) (layer "F.SilkS"))
  (fp_line (start -1.88 3.76) (end -1.08 3.76) (stroke (width 0.12) (type solid)) (layer "F.SilkS"))
  (pad "1" thru_hole rect (at 0 0 90) (size 2 2) (drill 1.2) (layers "*.Cu" "*.Mask") (remove_unused_layers no) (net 5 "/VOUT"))
  (pad "2" thru_hole circle (at 2.54 0 90) (size 2 2) (drill 1.2) (layers "*.Cu" "*.Mask") (remove_unused_layers no) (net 4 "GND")))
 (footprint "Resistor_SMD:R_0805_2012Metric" (layer "F.Cu") (at 61.52 81.53 90)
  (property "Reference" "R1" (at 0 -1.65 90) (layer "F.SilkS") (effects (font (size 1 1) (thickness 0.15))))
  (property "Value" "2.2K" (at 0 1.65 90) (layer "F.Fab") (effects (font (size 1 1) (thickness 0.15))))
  (fp_line (start -0.227064 -0.735) (end 0.227064 -0.735) (stroke (width 0.12) (type solid)) (layer "F.SilkS"))
  (fp_line (start -0.227064 0.735) (end 0.227064 0.735) (stroke (width 0.12) (type solid)) (layer "F.SilkS"))
  (pad "1" smd roundrect (at -0.9125 0 90) (size 1.025 1.4) (layers "F.Cu" "F.Paste" "F.Mask") (roundrect_rratio 0.243902) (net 8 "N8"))
  (pad "2" smd roundrect (at 0.9125 0 90) (size 1.025 1.4) (layers "F.Cu" "F.Paste" "F.Mask") (roundrect_rratio 0.243902) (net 7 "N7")))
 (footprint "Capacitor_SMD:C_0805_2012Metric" (layer "F.Cu") (at 75.21 91.04)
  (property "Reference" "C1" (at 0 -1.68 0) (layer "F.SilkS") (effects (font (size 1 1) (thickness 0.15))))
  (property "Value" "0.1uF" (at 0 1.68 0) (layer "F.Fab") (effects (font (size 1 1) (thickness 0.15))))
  (fp_line (start -0.261252 -0.735) (end 0.261252 -0.735) (stroke (width 0.12) (type solid)) (layer "F.SilkS"))
  (fp_line (start -0.261252 0.735) (end 0.261252 0.735) (stroke (width 0.12) (type solid)) (layer "F.SilkS"))
  (pad "1" smd roundrect (at -0.95 0) (size 1 1.45) (layers "F.Cu" "F.Paste" "F.Mask") (roundrect_rratio 0.25) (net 1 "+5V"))
  (pad "2" smd roundrect (at 0.95 0) (size 1 1.45) (layers "F.Cu" "F.Paste" "F.Mask") (roundrect_rratio 0.25) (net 4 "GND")))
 (gr_rect (start 49.43 74.09) (end 87.64 119.1) (stroke (width 0.05) (type default)) (fill none) (layer "Edge.Cuts"))
 (via (at 56.1 100.12) (size 0.6) (drill 0.3) (layers "F.Cu" "B.Cu") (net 4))
 (via (at 58.875 97.695) (size 0.6) (drill 0.3) (layers "F.Cu" "B.Cu") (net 4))
 (via (at 60.91 76.18) (size 0.6) (drill 0.3) (layers "F.Cu" "B.Cu") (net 4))
 (via (at 53.325 97.695) (size 0.6) (drill 0.3) (layers "F.Cu" "B.Cu") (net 4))
 (via (at 76.16 91.04) (size 0.6) (drill 0.3) (layers "F.Cu" "B.Cu") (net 4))
 (via (at 56.1 90.97) (size 0.6) (drill 0.3) (layers "F.Cu" "B.Cu") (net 4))
 (via (at 58.875 102.545) (size 0.6) (drill 0.3) (layers "F.Cu" "B.Cu") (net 4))
 (via (at 76.4925 80.58) (size 0.6) (drill 0.3) (layers "F.Cu" "B.Cu") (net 4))
 (via (at 53.325 102.545) (size 0.6) (drill 0.3) (layers "F.Cu" "B.Cu") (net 4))
 (via (at 63.31 111.5) (size 0.6) (drill 0.3) (layers "F.Cu" "B.Cu") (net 4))
 (segment (start 50.15 104.908298) (end 58.541702 113.3) (width 0.7) (layer "F.Cu") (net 1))
 (segment (start 54.14 80.75) (end 52.548 82.342) (width 0.7) (layer "F.Cu") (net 1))
 (segment (start 50.15 93.52) (end 50.15 104.908298) (width 0.7) (layer "F.Cu") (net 1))
 (segment (start 81.8944 99.33) (end 74.26 91.6956) (width 0.7) (layer "F.Cu") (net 1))
 (segment (start 52.548 82.342) (end 52.548 90.818) (width 0.7) (layer "F.Cu") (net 1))
 (segment (start 73.45 113.3) (end 84.26 102.49) (width 0.7) (layer "F.Cu") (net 1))
 (segment (start 52.548 90.818) (end 52.7 90.97) (width 0.7) (layer "F.Cu") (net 1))
 (segment (start 84.26 102.49) (end 84.26 99.33) (width 0.7) (layer "F.Cu") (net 1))
 (segment (start 84.26 99.33) (end 81.8944 99.33) (width 0.7) (layer "F.Cu") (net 1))
 (segment (start 58.541702 113.3) (end 73.45 113.3) (width 0.7) (layer "F.Cu") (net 1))
 (segment (start 52.7 90.97) (end 50.15 93.52) (width 0.7) (layer "F.Cu") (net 1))
 (segment (start 74.26 91.6956) (end 74.26 91.04) (width 0.7) (layer "F.Cu") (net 1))
 (segment (start 61.52 77.47) (end 62.81 76.18) (width 0.7) (layer "F.Cu") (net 7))
 (segment (start 61.52 80.6175) (end 61.52 77.47) (width 0.7) (layer "F.Cu") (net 7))
 (segment (start 65.9 93.82) (end 71.41 99.33) (width 0.7) (layer "F.Cu") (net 2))
 (segment (start 54.95 93.82) (end 63.0255 93.82) (width 0.7) (layer "F.Cu") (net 2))
 (segment (start 63.0255 93.82) (end 63.0255 84.012) (width 0.7) (layer "F.Cu") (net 2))
 (segment (start 54.4 90.97) (end 54.4 93.27) (width 0.7) (layer "F.Cu") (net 2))
 (segment (start 54.4 93.27) (end 54.95 93.82) (width 0.7) (layer "F.Cu") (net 2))
 (segment (start 71.41 99.33) (end 74.56 99.33) (width 0.7) (layer "F.Cu") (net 2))
 (segment (start 63.0255 84.012) (end 65.4275 81.61) (width 0.7) (layer "F.Cu") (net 2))
 (segment (start 63.0255 93.82) (end 65.9 93.82) (width 0.7) (layer "F.Cu") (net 2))
 (segment (start 76.8625 88.43) (end 76.1125 87.68) (width 0.7) (layer "F.Cu") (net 6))
 (segment (start 81.265 88.43) (end 76.8625 88.43) (width 0.7) (layer "F.Cu") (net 6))
 (segment (start 63.3547 74.8411) (end 60.3187 74.8411) (width 0.7) (layer "F.Cu") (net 3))
 (segment (start 57.8 77.3598) (end 57.8 90.97) (width 0.7) (layer "F.Cu") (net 3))
 (segment (start 67.8659 79.3523) (end 63.3547 74.8411) (width 0.7) (layer "F.Cu") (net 3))
 (segment (start 67.8659 80.1175) (end 74.205 80.1175) (width 0.7) (layer "F.Cu") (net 3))
 (segment (start 67.2 90.94) (end 67.2 89.44) (width 0.7) (layer "F.Cu") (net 3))
 (segment (start 67.3733 80.6101) (end 67.8659 80.1175) (width 0.7) (layer "F.Cu") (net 3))
 (segment (start 60.3187 74.8411) (end 57.8 77.3598) (width 0.7) (layer "F.Cu") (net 3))
 (segment (start 67.8659 80.1175) (end 67.8659 79.3523) (width 0.7) (layer "F.Cu") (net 3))
 (segment (start 74.205 80.1175) (end 74.6675 80.58) (width 0.7) (layer "F.Cu") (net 3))
 (segment (start 67.3733 89.2667) (end 67.3733 80.6101) (width 0.7) (layer "F.Cu") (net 3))
 (segment (start 67.2 89.44) (end 67.3733 89.2667) (width 0.7) (layer "F.Cu") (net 3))
 (segment (start 59.5 84.4625) (end 59.5 90.97) (width 0.7) (layer "F.Cu") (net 8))
 (segment (start 61.52 82.4425) (end 59.5 84.4625) (width 0.7) (layer "F.Cu") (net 8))
 (segment (start 71.2457 90.94) (end 70.75 90.94) (width 0.7) (layer "F.Cu") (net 5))
 (segment (start 76.5617 106.2483) (end 76.5617 96.256) (width 0.7) (layer "F.Cu") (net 5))
 (segment (start 71.2457 90.7218) (end 74.2875 87.68) (width 0.7) (layer "F.Cu") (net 5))
 (segment (start 74.2875 85.915) (end 73.7325 85.915) (width 0.7) (layer "F.Cu") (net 5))
 (segment (start 74.2875 85.915) (end 74.2875 87.68) (width 0.7) (layer "F.Cu") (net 5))
 (segment (start 69.5 90.94) (end 70.125 90.94) (width 0.7) (layer "F.Cu") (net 5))
 (segment (start 76.5617 96.256) (end 71.2457 90.94) (width 0.7) (layer "F.Cu") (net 5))
 (segment (start 71.31 111.5) (end 76.5617 106.2483) (width 0.7) (layer "F.Cu") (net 5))
 (segment (start 68.35 93.84) (end 68.35 92.34) (width 0.7) (layer "F.Cu") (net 5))
 (segment (start 76.7325 83.47) (end 74.2875 85.915) (width 0.7) (layer "F.Cu") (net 5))
 (segment (start 83.74 83.47) (end 76.7325 83.47) (width 0.7) (layer "F.Cu") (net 5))
 (segment (start 70.125 90.94) (end 68.725 92.34) (width 0.7) (layer "F.Cu") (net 5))
 (segment (start 71.2457 90.94) (end 71.2457 90.7218) (width 0.7) (layer "F.Cu") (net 5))
 (segment (start 70.125 90.94) (end 70.75 90.94) (width 0.7) (layer "F.Cu") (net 5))
 (segment (start 73.7325 85.915) (end 69.4275 81.61) (width 0.7) (layer "F.Cu") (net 5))
 (segment (start 68.725 92.34) (end 68.35 92.34) (width 0.7) (layer "F.Cu") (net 5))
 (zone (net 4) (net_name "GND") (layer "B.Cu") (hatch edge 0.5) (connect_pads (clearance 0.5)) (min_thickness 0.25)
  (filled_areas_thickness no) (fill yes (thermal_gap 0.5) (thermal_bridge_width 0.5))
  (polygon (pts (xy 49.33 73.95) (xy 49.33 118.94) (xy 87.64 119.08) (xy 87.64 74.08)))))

